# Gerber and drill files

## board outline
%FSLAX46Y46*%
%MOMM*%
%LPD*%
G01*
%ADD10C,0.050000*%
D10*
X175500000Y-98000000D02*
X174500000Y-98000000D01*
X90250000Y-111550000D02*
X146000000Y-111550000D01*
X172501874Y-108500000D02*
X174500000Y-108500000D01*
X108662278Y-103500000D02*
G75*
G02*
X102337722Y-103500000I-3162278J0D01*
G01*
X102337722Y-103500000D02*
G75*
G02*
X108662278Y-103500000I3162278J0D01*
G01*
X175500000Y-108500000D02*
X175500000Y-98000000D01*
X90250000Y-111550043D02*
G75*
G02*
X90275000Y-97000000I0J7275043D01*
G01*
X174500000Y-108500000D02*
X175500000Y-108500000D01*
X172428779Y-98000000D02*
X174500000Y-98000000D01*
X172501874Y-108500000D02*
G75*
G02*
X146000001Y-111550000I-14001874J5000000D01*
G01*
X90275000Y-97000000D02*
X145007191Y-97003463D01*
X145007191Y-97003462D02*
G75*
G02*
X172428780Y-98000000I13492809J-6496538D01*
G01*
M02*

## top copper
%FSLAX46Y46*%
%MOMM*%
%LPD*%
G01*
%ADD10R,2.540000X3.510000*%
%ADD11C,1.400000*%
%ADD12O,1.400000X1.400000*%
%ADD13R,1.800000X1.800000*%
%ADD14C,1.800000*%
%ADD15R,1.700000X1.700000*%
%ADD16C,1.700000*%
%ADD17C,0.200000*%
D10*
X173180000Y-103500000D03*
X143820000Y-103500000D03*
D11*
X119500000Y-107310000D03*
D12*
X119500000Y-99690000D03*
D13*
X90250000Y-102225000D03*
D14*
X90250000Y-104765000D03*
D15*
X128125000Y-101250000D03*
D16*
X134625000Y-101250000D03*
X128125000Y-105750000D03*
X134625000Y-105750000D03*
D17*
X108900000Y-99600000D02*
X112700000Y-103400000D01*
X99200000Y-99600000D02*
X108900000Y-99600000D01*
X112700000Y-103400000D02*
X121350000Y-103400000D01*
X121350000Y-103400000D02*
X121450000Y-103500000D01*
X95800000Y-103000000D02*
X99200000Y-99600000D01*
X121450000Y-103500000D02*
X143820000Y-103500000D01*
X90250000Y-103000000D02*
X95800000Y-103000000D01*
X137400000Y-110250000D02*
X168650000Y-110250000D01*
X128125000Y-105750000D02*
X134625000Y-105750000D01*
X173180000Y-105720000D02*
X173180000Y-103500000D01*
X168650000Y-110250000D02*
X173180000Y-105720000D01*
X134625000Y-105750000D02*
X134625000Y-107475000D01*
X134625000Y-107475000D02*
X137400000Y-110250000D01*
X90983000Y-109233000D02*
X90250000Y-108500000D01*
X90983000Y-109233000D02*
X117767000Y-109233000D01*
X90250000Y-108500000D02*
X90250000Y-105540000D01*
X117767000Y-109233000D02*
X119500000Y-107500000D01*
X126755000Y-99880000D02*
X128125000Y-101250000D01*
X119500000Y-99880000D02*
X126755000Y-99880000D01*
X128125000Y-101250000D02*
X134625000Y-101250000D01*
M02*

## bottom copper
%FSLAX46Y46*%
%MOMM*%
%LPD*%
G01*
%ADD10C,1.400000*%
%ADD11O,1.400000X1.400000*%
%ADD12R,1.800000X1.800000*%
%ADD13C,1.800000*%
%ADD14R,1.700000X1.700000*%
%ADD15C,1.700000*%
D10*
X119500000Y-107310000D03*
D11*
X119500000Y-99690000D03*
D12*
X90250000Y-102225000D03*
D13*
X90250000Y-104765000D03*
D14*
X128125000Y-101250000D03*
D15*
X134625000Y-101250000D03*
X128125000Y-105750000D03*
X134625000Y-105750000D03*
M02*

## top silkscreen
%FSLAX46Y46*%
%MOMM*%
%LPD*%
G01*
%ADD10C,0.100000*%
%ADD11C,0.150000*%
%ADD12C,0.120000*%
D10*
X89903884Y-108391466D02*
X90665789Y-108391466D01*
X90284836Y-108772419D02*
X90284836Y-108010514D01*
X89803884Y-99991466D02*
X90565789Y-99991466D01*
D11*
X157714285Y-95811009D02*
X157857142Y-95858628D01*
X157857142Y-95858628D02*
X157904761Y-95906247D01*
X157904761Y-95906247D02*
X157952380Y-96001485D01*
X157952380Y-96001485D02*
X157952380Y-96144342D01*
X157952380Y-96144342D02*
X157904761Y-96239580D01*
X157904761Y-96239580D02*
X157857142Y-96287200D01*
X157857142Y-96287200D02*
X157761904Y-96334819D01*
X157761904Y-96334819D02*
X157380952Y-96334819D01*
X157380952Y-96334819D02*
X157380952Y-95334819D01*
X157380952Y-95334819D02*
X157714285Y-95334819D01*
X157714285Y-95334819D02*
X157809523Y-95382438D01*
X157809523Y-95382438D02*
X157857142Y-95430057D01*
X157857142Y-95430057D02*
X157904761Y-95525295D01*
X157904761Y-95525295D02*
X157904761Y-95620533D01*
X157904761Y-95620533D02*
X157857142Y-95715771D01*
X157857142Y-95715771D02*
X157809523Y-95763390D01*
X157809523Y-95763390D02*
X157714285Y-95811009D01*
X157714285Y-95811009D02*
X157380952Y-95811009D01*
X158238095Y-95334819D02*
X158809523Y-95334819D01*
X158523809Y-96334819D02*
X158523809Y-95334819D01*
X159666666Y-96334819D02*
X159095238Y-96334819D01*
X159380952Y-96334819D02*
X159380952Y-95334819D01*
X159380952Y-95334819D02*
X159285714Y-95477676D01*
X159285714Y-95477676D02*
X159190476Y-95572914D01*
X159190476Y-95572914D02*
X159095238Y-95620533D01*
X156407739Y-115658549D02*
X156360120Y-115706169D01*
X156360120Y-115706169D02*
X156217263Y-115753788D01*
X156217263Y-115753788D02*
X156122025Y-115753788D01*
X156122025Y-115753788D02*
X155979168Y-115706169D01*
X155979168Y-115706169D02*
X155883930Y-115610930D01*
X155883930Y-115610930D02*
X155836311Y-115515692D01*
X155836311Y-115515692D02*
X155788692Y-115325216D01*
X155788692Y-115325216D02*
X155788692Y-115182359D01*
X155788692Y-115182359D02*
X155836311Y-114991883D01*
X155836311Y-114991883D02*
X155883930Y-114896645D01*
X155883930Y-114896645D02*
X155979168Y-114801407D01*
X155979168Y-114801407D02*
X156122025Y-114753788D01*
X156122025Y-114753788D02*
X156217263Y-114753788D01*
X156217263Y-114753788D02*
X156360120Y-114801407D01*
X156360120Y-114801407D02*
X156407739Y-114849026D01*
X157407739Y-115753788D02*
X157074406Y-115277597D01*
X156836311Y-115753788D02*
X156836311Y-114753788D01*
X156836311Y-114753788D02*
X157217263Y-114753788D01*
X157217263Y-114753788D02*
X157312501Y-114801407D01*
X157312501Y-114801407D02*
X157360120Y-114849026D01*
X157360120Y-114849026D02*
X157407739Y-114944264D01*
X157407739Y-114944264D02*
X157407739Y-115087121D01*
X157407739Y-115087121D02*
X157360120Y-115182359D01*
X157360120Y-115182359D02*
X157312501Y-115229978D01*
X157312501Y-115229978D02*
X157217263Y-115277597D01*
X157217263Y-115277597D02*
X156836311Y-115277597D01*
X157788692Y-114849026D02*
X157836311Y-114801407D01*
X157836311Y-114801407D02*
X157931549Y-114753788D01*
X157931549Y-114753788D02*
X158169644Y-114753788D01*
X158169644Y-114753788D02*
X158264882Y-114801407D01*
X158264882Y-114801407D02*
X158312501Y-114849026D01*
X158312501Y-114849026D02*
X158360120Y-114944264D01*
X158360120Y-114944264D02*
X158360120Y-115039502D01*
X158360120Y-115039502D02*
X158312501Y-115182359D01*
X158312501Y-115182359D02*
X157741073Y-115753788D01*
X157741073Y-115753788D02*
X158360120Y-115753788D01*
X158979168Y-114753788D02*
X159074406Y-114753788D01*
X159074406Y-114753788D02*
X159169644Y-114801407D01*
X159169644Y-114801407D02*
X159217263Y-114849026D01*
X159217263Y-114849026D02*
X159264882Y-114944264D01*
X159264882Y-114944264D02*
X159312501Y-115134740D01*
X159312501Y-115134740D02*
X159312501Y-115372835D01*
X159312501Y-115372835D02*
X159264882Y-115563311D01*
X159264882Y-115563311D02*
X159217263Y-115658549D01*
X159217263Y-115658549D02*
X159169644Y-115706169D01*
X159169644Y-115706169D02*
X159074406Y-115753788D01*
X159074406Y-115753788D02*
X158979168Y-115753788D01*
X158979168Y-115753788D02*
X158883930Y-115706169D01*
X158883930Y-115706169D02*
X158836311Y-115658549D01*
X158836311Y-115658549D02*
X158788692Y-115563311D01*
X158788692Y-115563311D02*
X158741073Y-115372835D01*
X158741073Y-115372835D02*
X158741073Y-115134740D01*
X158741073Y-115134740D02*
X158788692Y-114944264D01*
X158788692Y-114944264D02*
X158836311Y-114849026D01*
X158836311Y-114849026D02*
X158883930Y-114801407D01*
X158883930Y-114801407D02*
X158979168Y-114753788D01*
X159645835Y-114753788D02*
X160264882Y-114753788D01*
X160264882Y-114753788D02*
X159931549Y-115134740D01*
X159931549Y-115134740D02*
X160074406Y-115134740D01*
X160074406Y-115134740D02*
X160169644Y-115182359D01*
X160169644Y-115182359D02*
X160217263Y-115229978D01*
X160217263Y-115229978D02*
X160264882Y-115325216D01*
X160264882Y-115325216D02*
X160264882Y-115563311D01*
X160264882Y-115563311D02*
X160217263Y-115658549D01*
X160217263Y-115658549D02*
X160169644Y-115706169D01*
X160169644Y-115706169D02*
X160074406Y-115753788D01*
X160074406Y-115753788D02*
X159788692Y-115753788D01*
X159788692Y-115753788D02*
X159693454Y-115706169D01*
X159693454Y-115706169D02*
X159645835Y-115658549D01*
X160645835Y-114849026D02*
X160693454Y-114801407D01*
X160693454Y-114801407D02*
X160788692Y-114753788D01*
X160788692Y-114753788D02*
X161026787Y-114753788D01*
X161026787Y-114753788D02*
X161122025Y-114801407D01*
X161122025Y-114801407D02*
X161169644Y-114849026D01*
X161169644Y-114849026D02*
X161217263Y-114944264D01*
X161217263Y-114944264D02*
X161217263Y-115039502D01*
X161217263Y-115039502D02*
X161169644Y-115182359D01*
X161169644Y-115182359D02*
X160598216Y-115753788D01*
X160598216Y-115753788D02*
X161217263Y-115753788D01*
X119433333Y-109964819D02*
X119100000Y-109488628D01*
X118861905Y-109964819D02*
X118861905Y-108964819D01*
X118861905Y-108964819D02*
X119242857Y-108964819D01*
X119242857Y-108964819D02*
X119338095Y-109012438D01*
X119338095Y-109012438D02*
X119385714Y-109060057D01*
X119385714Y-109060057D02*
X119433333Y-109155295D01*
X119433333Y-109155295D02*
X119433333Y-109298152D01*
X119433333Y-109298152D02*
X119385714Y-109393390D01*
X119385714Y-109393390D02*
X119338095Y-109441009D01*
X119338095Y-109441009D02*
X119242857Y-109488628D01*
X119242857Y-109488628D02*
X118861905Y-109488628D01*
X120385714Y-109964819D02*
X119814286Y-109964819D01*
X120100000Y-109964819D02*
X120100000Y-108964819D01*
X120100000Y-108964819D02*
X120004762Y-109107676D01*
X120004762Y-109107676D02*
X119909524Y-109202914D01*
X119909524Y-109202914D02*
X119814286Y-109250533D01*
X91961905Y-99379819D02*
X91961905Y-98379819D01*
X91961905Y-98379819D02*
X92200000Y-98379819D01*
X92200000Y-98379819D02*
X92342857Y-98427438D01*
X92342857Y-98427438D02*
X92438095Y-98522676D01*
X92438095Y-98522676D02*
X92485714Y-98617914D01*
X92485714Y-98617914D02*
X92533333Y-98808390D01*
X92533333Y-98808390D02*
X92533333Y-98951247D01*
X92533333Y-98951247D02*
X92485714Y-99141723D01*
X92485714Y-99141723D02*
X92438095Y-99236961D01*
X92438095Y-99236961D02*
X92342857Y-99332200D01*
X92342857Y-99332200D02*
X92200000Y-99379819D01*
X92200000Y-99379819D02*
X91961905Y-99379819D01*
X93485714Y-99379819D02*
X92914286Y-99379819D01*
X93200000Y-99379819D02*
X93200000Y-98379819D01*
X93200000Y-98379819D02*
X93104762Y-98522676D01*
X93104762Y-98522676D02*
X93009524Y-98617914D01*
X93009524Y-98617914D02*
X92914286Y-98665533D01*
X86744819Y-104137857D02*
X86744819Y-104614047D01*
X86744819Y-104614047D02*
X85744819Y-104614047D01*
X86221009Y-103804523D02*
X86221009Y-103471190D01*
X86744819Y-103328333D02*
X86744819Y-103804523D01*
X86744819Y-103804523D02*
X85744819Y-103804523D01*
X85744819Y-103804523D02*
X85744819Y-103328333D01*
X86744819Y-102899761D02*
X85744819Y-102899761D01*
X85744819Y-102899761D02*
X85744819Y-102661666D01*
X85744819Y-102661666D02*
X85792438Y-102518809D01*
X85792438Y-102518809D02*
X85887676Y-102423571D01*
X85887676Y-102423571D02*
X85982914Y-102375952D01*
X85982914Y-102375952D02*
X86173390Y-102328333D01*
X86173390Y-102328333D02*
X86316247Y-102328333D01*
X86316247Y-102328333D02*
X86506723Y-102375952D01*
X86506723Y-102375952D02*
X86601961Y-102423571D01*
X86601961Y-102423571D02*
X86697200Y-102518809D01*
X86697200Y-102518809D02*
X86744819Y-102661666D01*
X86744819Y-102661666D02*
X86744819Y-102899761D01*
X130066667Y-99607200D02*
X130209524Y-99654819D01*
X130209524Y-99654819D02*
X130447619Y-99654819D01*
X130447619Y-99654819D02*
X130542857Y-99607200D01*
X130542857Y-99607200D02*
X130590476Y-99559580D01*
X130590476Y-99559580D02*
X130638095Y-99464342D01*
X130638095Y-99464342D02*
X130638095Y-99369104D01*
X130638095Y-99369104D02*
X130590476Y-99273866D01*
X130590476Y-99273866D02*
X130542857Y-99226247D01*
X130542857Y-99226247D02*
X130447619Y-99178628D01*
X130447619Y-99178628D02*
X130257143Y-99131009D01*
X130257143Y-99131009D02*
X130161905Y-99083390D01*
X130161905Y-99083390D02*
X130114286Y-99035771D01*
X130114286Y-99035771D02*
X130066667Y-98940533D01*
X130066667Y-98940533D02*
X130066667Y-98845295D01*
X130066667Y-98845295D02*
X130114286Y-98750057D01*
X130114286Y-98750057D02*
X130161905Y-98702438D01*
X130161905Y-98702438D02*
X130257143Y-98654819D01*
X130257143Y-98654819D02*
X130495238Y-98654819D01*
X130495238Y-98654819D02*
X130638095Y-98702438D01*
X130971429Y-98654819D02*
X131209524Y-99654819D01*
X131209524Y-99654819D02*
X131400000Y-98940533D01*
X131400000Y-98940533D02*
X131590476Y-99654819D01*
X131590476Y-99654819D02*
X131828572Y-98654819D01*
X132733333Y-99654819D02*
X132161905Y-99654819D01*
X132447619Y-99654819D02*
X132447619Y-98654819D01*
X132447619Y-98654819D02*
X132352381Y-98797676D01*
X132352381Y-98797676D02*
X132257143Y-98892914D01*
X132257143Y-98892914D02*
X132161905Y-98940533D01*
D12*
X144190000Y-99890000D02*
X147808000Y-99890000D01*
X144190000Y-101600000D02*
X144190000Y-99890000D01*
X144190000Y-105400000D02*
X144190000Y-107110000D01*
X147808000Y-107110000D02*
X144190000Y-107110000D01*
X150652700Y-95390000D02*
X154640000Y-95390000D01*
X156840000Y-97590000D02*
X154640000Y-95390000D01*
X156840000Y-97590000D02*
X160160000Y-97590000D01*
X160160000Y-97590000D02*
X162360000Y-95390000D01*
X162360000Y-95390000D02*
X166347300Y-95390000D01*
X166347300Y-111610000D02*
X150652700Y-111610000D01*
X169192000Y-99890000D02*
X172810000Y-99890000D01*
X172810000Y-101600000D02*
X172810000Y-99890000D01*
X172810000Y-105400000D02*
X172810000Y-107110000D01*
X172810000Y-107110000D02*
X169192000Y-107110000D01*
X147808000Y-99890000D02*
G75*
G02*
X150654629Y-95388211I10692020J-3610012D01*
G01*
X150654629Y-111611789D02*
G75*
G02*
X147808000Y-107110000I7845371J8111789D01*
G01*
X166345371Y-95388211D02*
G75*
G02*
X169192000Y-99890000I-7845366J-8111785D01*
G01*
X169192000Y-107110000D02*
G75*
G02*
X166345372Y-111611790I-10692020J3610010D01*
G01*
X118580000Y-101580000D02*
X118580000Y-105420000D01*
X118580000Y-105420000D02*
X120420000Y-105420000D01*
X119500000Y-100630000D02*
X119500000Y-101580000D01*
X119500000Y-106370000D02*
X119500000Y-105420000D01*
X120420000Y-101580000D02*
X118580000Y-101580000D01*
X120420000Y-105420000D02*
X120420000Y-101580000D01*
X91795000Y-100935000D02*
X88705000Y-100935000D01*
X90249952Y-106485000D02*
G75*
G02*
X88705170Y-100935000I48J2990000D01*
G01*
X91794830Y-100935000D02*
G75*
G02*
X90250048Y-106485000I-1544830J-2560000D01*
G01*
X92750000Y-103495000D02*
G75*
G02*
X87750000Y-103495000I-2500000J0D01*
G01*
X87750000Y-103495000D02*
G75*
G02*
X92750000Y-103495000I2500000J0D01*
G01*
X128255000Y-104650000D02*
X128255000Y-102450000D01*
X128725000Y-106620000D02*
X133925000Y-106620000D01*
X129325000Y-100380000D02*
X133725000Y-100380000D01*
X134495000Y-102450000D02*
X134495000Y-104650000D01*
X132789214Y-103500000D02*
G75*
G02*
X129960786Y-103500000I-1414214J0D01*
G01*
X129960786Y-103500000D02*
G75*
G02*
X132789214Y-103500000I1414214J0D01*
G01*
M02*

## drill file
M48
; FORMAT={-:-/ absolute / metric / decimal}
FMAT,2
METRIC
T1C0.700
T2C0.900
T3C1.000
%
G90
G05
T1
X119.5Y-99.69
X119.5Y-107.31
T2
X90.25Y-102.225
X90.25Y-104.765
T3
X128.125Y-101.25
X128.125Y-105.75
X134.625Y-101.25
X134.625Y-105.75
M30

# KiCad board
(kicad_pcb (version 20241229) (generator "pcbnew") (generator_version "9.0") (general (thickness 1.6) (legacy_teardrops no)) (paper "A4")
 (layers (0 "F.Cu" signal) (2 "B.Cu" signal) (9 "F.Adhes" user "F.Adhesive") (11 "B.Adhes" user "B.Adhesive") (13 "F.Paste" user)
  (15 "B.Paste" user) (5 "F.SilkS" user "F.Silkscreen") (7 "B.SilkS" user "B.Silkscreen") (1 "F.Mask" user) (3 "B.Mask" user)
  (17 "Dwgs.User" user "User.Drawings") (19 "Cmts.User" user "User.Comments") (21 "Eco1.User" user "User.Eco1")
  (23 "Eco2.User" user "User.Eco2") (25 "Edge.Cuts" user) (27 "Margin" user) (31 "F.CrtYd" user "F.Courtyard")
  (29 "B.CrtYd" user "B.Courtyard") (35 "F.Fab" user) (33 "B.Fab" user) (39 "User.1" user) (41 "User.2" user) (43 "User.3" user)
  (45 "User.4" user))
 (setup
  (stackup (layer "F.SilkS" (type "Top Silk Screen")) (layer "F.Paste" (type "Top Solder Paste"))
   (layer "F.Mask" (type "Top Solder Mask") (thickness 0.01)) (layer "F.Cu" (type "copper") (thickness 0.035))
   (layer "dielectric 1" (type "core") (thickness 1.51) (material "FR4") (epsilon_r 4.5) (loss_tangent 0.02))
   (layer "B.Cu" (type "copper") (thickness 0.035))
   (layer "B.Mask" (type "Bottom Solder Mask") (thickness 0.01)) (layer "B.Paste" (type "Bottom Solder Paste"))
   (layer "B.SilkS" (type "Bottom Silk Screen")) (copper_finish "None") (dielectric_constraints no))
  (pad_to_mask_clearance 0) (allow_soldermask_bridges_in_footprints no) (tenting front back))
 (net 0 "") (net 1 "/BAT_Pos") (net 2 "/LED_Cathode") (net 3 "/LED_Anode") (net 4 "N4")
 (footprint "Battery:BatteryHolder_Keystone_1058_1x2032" (layer "F.Cu") (at 158.5 103.5 180)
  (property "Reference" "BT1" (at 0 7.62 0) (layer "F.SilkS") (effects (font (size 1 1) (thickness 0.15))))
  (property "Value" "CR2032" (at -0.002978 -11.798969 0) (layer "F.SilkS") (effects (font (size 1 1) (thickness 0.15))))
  (fp_line (start 14.31 3.61) (end 10.692 3.61) (stroke (width 0.12) (type solid)) (layer "F.SilkS"))
  (fp_line (start 14.31 1.9) (end 14.31 3.61) (stroke (width 0.12) (type solid)) (layer "F.SilkS"))
  (fp_line (start 14.31 -1.9) (end 14.31 -3.61) (stroke (width 0.12) (type solid)) (layer "F.SilkS"))
  (fp_line (start 10.692 -3.61) (end 14.31 -3.61) (stroke (width 0.12) (type solid)) (layer "F.SilkS"))
  (fp_line (start 7.8473 8.11) (end 3.86 8.11) (stroke (width 0.12) (type solid)) (layer "F.SilkS"))
  (fp_line (start 1.66 5.91) (end 3.86 8.11) (stroke (width 0.12) (type solid)) (layer "F.SilkS"))
  (fp_line (start 1.66 5.91) (end -1.66 5.91) (stroke (width 0.12) (type solid)) (layer "F.SilkS"))
  (fp_line (start -1.66 5.91) (end -3.86 8.11) (stroke (width 0.12) (type solid)) (layer "F.SilkS"))
  (fp_line (start -3.86 8.11) (end -7.8473 8.11) (stroke (width 0.12) (type solid)) (layer "F.SilkS"))
  (fp_line (start -7.8473 -8.11) (end 7.8473 -8.11) (stroke (width 0.12) (type solid)) (layer "F.SilkS"))
  (fp_line (start -10.692 3.61) (end -14.31 3.61) (stroke (width 0.12) (type solid)) (layer "F.SilkS"))
  (fp_line (start -14.31 1.9) (end -14.31 3.61) (stroke (width 0.12) (type solid)) (layer "F.SilkS"))
  (fp_line (start -14.31 -1.9) (end -14.31 -3.61) (stroke (width 0.12) (type solid)) (layer "F.SilkS"))
  (fp_line (start -14.31 -3.61) (end -10.692 -3.61) (stroke (width 0.12) (type solid)) (layer "F.SilkS"))
  (fp_arc (start 10.692 3.61) (mid 9.538084 6.031244) (end 7.845371 8.111789) (stroke (width 0.12) (type solid)) (layer "F.SilkS"))
  (fp_arc (start 7.845371 -8.111789) (mid 9.538085 -6.031244) (end 10.692 -3.61) (stroke (width 0.12) (type solid)) (layer "F.SilkS"))
  (fp_arc (start -7.845371 8.111789) (mid -9.538085 6.031244) (end -10.692 3.61) (stroke (width 0.12) (type solid)) (layer "F.SilkS"))
  (fp_arc (start -10.692 -3.61) (mid -9.538084 -6.031244) (end -7.845371 -8.111789) (stroke (width 0.12) (type solid)) (layer "F.SilkS"))
  (pad "1" smd rect (at -14.68 0 180) (size 2.54 3.51) (layers "F.Cu" "F.Mask" "F.Paste") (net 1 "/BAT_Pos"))
  (pad "2" smd rect (at 14.68 0 180) (size 2.54 3.51) (layers "F.Cu" "F.Mask" "F.Paste") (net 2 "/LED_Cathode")))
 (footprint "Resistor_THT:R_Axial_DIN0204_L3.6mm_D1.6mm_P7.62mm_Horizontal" (layer "F.Cu") (at 119.5 107.31 90)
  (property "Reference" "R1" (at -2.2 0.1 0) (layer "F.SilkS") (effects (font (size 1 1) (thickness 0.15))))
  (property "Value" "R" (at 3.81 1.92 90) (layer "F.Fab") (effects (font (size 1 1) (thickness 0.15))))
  (fp_line (start 5.73 -0.92) (end 1.89 -0.92) (stroke (width 0.12) (type solid)) (layer "F.SilkS"))
  (fp_line (start 1.89 -0.92) (end 1.89 0.92) (stroke (width 0.12) (type solid)) (layer "F.SilkS"))
  (fp_line (start 6.68 0) (end 5.73 0) (stroke (width 0.12) (type solid)) (layer "F.SilkS"))
  (fp_line (start 0.94 0) (end 1.89 0) (stroke (width 0.12) (type solid)) (layer "F.SilkS"))
  (fp_line (start 5.73 0.92) (end 5.73 -0.92) (stroke (width 0.12) (type solid)) (layer "F.SilkS"))
  (fp_line (start 1.89 0.92) (end 5.73 0.92) (stroke (width 0.12) (type solid)) (layer "F.SilkS"))
  (pad "1" thru_hole circle (at 0 0 90) (size 1.4 1.4) (drill 0.7) (layers "*.Cu" "*.Mask") (remove_unused_layers no) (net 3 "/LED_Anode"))
  (pad "2" thru_hole oval (at 7.62 0 90) (size 1.4 1.4) (drill 0.7) (layers "*.Cu" "*.Mask") (remove_unused_layers no) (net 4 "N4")))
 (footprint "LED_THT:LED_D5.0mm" (layer "F.Cu") (at 90.25 102.225 -90)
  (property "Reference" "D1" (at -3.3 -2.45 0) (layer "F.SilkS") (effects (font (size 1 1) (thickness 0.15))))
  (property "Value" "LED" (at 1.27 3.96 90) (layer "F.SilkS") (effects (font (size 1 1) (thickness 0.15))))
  (fp_line (start -1.29 -1.545) (end -1.29 1.545) (stroke (width 0.12) (type solid)) (layer "F.SilkS"))
  (fp_arc (start 4.26 0.000048) (mid 2.071756 2.880501) (end -1.29 1.54483) (stroke (width 0.12) (type solid)) (layer "F.SilkS"))
  (fp_arc (start -1.29 -1.54483) (mid 2.071756 -2.880501) (end 4.26 -0.000048) (stroke (width 0.12) (type solid)) (layer "F.SilkS"))
  (fp_circle (center 1.27 0) (end 3.77 0) (stroke (width 0.12) (type solid)) (fill no) (layer "F.SilkS"))
  (pad "1" thru_hole rect (at 0 0 270) (size 1.8 1.8) (drill 0.9) (layers "*.Cu" "*.Mask") (remove_unused_layers no) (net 2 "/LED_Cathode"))
  (pad "2" thru_hole circle (at 2.54 0 270) (size 1.8 1.8) (drill 0.9) (layers "*.Cu" "*.Mask") (remove_unused_layers no)
   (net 3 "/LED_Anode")))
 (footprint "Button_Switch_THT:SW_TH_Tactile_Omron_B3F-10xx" (layer "F.Cu") (at 128.125 101.25)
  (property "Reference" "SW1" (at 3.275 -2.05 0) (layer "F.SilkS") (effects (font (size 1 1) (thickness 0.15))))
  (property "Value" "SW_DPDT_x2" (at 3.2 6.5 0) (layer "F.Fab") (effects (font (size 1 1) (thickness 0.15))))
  (fp_line (start 0.13 3.4) (end 0.13 1.2) (stroke (width 0.12) (type solid)) (layer "F.SilkS"))
  (fp_line (start 0.6 5.37) (end 5.8 5.37) (stroke (width 0.12) (type solid)) (layer "F.SilkS"))
  (fp_line (start 1.2 -0.87) (end 5.6 -0.87) (stroke (width 0.12) (type solid)) (layer "F.SilkS"))
  (fp_line (start 6.37 1.2) (end 6.37 3.4) (stroke (width 0.12) (type solid)) (layer "F.SilkS"))
  (fp_circle (center 3.25 2.25) (end 4.25 3.25) (stroke (width 0.12) (type solid)) (fill no) (layer "F.SilkS"))
  (pad "1" thru_hole rect (at 0 0) (size 1.7 1.7) (drill 1) (layers "*.Cu" "*.Mask") (remove_unused_layers no) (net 4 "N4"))
  (pad "1" thru_hole circle (at 6.5 0) (size 1.7 1.7) (drill 1) (layers "*.Cu" "*.Mask") (remove_unused_layers no) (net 4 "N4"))
  (pad "2" thru_hole circle (at 0 4.5) (size 1.7 1.7) (drill 1) (layers "*.Cu" "*.Mask") (remove_unused_layers no) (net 1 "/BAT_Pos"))
  (pad "2" thru_hole circle (at 6.5 4.5) (size 1.7 1.7) (drill 1) (layers "*.Cu" "*.Mask") (remove_unused_layers no) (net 1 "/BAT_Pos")))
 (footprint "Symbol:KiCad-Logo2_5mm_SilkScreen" (layer "B.Cu") (at 158.5 103.48729 180)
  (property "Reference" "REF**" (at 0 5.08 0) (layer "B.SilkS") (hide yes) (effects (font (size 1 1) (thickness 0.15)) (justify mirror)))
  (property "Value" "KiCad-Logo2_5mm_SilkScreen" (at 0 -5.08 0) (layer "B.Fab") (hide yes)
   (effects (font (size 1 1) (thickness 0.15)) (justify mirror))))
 (gr_line (start 175.5 98) (end 174.5 98) (stroke (width 0.05) (type default)) (locked yes) (layer "Edge.Cuts"))
 (gr_line (start 90.25 111.55) (end 146 111.55) (stroke (width 0.05) (type default)) (locked yes) (layer "Edge.Cuts"))
 (gr_line (start 172.501874 108.5) (end 174.5 108.5) (stroke (width 0.05) (type default)) (locked yes) (layer "Edge.Cuts"))
 (gr_circle (center 105.5 103.5) (end 108.5 102.5) (stroke (width 0.05) (type default)) (fill no) (layer "Edge.Cuts"))
 (gr_line (start 175.5 108.5) (end 175.5 98) (stroke (width 0.05) (type default)) (locked yes) (layer "Edge.Cuts"))
 (gr_arc (start 90.25 111.550043) (mid 82.974968 104.2625) (end 90.275 97) (stroke (width 0.05) (type default)) (locked yes)
  (layer "Edge.Cuts"))
 (gr_line (start 174.5 108.5) (end 175.5 108.5) (stroke (width 0.05) (type default)) (locked yes) (layer "Edge.Cuts"))
 (gr_line (start 172.428779 98) (end 174.5 98) (stroke (width 0.05) (type default)) (locked yes) (layer "Edge.Cuts"))
 (gr_arc (start 172.501874 108.5) (mid 160.199862 118.27034) (end 146 111.55) (stroke (width 0.05) (type default)) (locked yes)
  (layer "Edge.Cuts"))
 (gr_line (start 90.275 97) (end 145.007191 97.003463) (stroke (width 0.05) (type default)) (locked yes) (layer "Edge.Cuts"))
 (gr_arc (start 145.007191 97.003462) (mid 159.043865 88.534536) (end 172.428779 98) (stroke (width 0.05) (type default)) (locked yes)
  (layer "Edge.Cuts"))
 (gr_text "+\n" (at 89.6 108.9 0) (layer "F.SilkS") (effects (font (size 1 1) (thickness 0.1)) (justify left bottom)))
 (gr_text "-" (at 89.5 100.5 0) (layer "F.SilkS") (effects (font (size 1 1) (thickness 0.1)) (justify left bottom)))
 (segment (start 108.9 99.6) (end 112.7 103.4) (width 0.2) (layer "F.Cu") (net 2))
 (segment (start 99.2 99.6) (end 108.9 99.6) (width 0.2) (layer "F.Cu") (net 2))
 (segment (start 112.7 103.4) (end 121.35 103.4) (width 0.2) (layer "F.Cu") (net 2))
 (segment (start 121.35 103.4) (end 121.45 103.5) (width 0.2) (layer "F.Cu") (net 2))
 (segment (start 95.8 103) (end 99.2 99.6) (width 0.2) (layer "F.Cu") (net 2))
 (segment (start 121.45 103.5) (end 143.82 103.5) (width 0.2) (layer "F.Cu") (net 2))
 (segment (start 90.25 103) (end 95.8 103) (width 0.2) (layer "F.Cu") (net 2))
 (segment (start 137.4 110.25) (end 168.65 110.25) (width 0.2) (layer "F.Cu") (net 1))
 (segment (start 128.125 105.75) (end 134.625 105.75) (width 0.2) (layer "F.Cu") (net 1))
 (segment (start 173.18 105.72) (end 173.18 103.5) (width 0.2) (layer "F.Cu") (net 1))
 (segment (start 168.65 110.25) (end 173.18 105.72) (width 0.2) (layer "F.Cu") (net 1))
 (segment (start 134.625 105.75) (end 134.625 107.475) (width 0.2) (layer "F.Cu") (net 1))
 (segment (start 134.625 107.475) (end 137.4 110.25) (width 0.2) (layer "F.Cu") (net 1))
 (segment (start 90.983 109.233) (end 90.25 108.5) (width 0.2) (layer "F.Cu") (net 3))
 (segment (start 90.983 109.233) (end 117.767 109.233) (width 0.2) (layer "F.Cu") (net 3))
 (segment (start 90.25 108.5) (end 90.25 105.54) (width 0.2) (layer "F.Cu") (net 3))
 (segment (start 117.767 109.233) (end 119.5 107.5) (width 0.2) (layer "F.Cu") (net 3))
 (segment (start 126.755 99.88) (end 128.125 101.25) (width 0.2) (layer "F.Cu") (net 4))
 (segment (start 119.5 99.88) (end 126.755 99.88) (width 0.2) (layer "F.Cu") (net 4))
 (segment (start 128.125 101.25) (end 134.625 101.25) (width 0.2) (layer "F.Cu") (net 4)))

